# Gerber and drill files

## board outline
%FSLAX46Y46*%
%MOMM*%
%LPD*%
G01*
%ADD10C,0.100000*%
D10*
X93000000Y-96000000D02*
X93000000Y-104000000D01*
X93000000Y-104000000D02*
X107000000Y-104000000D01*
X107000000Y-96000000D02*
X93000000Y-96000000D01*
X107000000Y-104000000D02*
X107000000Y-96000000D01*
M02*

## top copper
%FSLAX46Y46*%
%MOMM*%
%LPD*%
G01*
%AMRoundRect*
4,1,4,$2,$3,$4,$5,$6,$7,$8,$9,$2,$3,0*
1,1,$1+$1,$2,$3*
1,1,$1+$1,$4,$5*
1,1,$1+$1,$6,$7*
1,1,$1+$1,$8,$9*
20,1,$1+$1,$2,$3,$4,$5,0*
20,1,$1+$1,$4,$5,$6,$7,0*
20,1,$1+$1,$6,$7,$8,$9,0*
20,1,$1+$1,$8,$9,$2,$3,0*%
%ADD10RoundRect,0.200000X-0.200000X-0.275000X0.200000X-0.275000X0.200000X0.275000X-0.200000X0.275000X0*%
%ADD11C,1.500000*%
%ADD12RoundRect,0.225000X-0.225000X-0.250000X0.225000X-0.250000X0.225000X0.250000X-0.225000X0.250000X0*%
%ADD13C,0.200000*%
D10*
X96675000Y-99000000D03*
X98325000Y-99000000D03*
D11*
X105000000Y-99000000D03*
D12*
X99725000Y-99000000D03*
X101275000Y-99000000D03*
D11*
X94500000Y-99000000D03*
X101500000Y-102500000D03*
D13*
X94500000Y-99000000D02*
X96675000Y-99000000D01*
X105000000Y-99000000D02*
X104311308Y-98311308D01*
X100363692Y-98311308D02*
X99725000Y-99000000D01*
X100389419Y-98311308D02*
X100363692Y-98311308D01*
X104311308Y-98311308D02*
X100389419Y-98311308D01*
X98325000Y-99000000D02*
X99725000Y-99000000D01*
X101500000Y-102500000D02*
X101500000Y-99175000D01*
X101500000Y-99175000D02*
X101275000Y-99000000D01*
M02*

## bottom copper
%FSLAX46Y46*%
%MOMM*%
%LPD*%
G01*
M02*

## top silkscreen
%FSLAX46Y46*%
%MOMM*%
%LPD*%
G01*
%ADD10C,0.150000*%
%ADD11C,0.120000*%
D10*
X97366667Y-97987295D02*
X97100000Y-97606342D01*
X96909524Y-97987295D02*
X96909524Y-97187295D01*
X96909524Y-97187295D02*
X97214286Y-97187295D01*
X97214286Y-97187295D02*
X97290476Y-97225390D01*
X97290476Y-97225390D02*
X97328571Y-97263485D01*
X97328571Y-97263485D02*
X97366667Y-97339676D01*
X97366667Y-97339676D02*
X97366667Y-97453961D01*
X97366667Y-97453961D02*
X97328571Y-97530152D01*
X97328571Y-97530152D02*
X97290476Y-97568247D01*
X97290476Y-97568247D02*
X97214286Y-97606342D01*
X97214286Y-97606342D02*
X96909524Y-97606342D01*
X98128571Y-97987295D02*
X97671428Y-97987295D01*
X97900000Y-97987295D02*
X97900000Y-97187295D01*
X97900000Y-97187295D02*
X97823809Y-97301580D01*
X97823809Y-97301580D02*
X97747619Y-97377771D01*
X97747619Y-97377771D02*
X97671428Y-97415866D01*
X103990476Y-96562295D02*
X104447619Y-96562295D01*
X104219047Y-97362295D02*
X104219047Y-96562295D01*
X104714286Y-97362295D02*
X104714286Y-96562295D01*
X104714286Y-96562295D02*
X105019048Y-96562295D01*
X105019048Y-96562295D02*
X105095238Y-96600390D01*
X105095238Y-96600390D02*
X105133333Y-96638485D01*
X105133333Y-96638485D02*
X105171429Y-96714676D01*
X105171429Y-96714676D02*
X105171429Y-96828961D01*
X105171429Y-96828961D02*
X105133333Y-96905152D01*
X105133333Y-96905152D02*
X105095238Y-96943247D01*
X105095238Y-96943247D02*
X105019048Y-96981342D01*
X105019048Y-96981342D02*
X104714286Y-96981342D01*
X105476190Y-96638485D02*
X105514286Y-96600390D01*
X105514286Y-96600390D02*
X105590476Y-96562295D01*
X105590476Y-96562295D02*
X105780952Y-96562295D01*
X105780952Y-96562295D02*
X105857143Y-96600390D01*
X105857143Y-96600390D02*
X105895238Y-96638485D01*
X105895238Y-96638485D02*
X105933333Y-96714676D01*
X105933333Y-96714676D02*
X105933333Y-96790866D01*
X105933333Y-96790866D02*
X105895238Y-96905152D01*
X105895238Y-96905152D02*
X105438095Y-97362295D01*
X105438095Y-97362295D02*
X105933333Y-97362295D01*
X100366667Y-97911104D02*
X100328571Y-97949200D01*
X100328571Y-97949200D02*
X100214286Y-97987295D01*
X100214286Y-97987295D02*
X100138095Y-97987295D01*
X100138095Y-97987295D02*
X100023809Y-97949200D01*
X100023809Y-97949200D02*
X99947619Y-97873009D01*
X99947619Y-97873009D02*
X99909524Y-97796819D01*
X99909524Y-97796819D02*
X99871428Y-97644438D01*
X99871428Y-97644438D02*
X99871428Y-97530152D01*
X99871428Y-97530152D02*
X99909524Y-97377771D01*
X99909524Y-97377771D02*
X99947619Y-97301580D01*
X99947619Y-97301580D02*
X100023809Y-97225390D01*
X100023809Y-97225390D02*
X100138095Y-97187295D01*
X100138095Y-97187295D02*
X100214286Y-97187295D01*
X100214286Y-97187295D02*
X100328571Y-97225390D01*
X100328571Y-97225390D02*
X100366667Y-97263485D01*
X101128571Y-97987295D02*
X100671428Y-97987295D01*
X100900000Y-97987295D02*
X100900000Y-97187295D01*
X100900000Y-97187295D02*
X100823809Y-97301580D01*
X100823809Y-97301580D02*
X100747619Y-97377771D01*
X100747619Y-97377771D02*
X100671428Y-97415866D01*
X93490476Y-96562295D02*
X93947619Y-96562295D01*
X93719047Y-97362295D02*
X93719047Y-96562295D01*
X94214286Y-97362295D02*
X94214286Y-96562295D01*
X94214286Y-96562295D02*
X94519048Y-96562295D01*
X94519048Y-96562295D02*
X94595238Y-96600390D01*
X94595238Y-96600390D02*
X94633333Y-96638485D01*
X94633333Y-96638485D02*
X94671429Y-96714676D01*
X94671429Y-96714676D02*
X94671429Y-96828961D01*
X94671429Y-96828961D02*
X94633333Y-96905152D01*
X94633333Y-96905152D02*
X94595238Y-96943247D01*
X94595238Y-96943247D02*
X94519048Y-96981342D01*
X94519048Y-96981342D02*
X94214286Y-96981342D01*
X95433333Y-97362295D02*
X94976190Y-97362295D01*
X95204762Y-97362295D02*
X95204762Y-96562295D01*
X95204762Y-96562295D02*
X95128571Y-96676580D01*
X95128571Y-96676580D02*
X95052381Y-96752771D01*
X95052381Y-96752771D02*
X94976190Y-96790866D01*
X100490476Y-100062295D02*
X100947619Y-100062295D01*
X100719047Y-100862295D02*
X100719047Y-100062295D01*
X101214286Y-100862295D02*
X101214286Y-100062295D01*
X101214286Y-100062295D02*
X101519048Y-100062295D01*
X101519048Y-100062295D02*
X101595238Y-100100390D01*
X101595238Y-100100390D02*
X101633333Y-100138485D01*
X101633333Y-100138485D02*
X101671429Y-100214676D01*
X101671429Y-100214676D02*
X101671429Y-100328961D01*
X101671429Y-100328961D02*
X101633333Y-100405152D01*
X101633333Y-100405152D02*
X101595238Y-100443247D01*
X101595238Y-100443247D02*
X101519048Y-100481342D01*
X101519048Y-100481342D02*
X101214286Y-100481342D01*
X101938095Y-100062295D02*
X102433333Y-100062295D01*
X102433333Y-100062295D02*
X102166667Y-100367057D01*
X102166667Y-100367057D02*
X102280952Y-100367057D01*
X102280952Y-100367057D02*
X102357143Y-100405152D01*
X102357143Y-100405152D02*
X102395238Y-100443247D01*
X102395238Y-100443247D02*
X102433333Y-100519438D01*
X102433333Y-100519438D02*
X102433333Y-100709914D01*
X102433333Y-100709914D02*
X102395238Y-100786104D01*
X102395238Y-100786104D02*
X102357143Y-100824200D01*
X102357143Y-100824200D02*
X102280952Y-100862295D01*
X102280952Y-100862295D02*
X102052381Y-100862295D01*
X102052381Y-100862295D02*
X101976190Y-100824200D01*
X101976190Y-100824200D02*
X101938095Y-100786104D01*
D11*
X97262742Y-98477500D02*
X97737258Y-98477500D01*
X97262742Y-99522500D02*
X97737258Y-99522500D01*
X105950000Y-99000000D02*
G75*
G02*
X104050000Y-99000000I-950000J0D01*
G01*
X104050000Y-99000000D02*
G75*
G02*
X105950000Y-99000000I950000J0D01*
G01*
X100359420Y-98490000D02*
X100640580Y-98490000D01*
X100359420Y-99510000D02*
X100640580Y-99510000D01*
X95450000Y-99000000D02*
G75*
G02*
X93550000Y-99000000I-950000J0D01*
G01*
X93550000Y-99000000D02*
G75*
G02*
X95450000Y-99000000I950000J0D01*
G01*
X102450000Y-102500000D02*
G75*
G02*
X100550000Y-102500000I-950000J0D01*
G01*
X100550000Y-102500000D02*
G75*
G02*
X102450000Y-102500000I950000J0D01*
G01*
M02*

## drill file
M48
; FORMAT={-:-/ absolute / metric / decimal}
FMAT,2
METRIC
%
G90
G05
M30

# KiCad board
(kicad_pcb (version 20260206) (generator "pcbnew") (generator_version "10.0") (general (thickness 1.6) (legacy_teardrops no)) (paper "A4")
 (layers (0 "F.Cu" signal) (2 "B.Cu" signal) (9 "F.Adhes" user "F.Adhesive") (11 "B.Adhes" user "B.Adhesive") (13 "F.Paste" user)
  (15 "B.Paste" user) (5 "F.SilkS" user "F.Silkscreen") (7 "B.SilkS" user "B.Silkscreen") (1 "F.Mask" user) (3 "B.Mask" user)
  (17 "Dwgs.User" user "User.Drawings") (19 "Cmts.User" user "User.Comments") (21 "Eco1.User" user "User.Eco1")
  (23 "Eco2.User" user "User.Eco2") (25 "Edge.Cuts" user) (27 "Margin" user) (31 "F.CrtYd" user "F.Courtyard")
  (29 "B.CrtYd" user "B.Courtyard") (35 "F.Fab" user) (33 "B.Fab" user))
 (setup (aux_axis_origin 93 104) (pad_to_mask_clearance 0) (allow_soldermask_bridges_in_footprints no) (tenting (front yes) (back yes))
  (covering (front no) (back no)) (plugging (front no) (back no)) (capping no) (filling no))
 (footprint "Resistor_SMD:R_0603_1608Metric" (layer "F.Cu") (at 97.5 99)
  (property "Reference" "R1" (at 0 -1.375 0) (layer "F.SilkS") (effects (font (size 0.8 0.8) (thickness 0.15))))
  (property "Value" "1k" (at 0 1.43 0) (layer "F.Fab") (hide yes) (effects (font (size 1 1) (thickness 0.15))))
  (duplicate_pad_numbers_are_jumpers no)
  (fp_line (start -0.237258 -0.5225) (end 0.237258 -0.5225) (stroke (width 0.12) (type solid)) (layer "F.SilkS"))
  (fp_line (start -0.237258 0.5225) (end 0.237258 0.5225) (stroke (width 0.12) (type solid)) (layer "F.SilkS"))
  (pad "1" smd roundrect (at -0.825 0) (size 0.8 0.95) (layers "F.Cu" "F.Mask" "F.Paste") (roundrect_rratio 0.25) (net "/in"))
  (pad "2" smd roundrect (at 0.825 0) (size 0.8 0.95) (layers "F.Cu" "F.Mask" "F.Paste") (roundrect_rratio 0.25) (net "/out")))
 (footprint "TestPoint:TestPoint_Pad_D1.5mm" (layer "F.Cu") (at 105 99)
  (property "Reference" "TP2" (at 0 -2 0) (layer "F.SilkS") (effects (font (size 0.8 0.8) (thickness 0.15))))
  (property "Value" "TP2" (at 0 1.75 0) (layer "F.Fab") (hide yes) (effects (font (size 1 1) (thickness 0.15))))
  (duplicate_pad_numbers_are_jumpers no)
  (fp_circle (center 0 0) (end 0 0.95) (stroke (width 0.12) (type solid)) (fill no) (layer "F.SilkS"))
  (pad "1" smd circle (at 0 0) (size 1.5 1.5) (layers "F.Cu" "F.Mask") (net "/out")))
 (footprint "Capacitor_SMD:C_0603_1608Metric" (layer "F.Cu") (at 100.5 99)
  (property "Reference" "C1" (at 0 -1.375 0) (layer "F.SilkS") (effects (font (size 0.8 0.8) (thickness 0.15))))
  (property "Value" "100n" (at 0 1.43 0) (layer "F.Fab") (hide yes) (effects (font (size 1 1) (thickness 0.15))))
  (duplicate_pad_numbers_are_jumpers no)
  (fp_line (start -0.14058 -0.51) (end 0.14058 -0.51) (stroke (width 0.12) (type solid)) (layer "F.SilkS"))
  (fp_line (start -0.14058 0.51) (end 0.14058 0.51) (stroke (width 0.12) (type solid)) (layer "F.SilkS"))
  (pad "1" smd roundrect (at -0.775 0) (size 0.9 0.95) (layers "F.Cu" "F.Mask" "F.Paste") (roundrect_rratio 0.25) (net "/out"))
  (pad "2" smd roundrect (at 0.775 0) (size 0.9 0.95) (layers "F.Cu" "F.Mask" "F.Paste") (roundrect_rratio 0.25) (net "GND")))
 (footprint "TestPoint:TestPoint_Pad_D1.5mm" (layer "F.Cu") (at 94.5 99)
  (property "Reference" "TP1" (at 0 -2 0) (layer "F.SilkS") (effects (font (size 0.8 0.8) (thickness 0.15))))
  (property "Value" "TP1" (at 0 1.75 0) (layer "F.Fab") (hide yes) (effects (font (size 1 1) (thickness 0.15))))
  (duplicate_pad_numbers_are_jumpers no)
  (fp_circle (center 0 0) (end 0 0.95) (stroke (width 0.12) (type solid)) (fill no) (layer "F.SilkS"))
  (pad "1" smd circle (at 0 0) (size 1.5 1.5) (layers "F.Cu" "F.Mask") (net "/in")))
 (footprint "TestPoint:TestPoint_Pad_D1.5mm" (layer "F.Cu") (at 101.5 102.5)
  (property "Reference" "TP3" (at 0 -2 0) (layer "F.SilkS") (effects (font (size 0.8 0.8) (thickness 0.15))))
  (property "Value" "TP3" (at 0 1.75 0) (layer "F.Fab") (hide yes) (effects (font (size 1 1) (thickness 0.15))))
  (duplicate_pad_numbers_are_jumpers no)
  (fp_circle (center 0 0) (end 0 0.95) (stroke (width 0.12) (type solid)) (fill no) (layer "F.SilkS"))
  (pad "1" smd circle (at 0 0) (size 1.5 1.5) (layers "F.Cu" "F.Mask") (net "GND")))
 (gr_line (start 93 96) (end 93 104) (stroke (width 0.1) (type solid)) (layer "Edge.Cuts"))
 (gr_line (start 93 104) (end 107 104) (stroke (width 0.1) (type solid)) (layer "Edge.Cuts"))
 (gr_line (start 107 96) (end 93 96) (stroke (width 0.1) (type solid)) (layer "Edge.Cuts"))
 (gr_line (start 107 104) (end 107 96) (stroke (width 0.1) (type solid)) (layer "Edge.Cuts"))
 (segment (start 94.5 99) (end 96.675 99) (width 0.2) (layer "F.Cu") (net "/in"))
 (segment (start 105 99) (end 104.311308 98.311308) (width 0.2) (layer "F.Cu") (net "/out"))
 (segment (start 100.363692 98.311308) (end 99.725 99) (width 0.2) (layer "F.Cu") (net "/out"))
 (segment (start 100.389419 98.311308) (end 100.363692 98.311308) (width 0.2) (layer "F.Cu") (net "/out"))
 (segment (start 104.311308 98.311308) (end 100.389419 98.311308) (width 0.2) (layer "F.Cu") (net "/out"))
 (segment (start 98.325 99) (end 99.725 99) (width 0.2) (layer "F.Cu") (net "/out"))
 (segment (start 101.5 102.5) (end 101.5 99.175) (width 0.2) (layer "F.Cu") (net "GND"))
 (segment (start 101.5 99.175) (end 101.275 99) (width 0.2) (layer "F.Cu") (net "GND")))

